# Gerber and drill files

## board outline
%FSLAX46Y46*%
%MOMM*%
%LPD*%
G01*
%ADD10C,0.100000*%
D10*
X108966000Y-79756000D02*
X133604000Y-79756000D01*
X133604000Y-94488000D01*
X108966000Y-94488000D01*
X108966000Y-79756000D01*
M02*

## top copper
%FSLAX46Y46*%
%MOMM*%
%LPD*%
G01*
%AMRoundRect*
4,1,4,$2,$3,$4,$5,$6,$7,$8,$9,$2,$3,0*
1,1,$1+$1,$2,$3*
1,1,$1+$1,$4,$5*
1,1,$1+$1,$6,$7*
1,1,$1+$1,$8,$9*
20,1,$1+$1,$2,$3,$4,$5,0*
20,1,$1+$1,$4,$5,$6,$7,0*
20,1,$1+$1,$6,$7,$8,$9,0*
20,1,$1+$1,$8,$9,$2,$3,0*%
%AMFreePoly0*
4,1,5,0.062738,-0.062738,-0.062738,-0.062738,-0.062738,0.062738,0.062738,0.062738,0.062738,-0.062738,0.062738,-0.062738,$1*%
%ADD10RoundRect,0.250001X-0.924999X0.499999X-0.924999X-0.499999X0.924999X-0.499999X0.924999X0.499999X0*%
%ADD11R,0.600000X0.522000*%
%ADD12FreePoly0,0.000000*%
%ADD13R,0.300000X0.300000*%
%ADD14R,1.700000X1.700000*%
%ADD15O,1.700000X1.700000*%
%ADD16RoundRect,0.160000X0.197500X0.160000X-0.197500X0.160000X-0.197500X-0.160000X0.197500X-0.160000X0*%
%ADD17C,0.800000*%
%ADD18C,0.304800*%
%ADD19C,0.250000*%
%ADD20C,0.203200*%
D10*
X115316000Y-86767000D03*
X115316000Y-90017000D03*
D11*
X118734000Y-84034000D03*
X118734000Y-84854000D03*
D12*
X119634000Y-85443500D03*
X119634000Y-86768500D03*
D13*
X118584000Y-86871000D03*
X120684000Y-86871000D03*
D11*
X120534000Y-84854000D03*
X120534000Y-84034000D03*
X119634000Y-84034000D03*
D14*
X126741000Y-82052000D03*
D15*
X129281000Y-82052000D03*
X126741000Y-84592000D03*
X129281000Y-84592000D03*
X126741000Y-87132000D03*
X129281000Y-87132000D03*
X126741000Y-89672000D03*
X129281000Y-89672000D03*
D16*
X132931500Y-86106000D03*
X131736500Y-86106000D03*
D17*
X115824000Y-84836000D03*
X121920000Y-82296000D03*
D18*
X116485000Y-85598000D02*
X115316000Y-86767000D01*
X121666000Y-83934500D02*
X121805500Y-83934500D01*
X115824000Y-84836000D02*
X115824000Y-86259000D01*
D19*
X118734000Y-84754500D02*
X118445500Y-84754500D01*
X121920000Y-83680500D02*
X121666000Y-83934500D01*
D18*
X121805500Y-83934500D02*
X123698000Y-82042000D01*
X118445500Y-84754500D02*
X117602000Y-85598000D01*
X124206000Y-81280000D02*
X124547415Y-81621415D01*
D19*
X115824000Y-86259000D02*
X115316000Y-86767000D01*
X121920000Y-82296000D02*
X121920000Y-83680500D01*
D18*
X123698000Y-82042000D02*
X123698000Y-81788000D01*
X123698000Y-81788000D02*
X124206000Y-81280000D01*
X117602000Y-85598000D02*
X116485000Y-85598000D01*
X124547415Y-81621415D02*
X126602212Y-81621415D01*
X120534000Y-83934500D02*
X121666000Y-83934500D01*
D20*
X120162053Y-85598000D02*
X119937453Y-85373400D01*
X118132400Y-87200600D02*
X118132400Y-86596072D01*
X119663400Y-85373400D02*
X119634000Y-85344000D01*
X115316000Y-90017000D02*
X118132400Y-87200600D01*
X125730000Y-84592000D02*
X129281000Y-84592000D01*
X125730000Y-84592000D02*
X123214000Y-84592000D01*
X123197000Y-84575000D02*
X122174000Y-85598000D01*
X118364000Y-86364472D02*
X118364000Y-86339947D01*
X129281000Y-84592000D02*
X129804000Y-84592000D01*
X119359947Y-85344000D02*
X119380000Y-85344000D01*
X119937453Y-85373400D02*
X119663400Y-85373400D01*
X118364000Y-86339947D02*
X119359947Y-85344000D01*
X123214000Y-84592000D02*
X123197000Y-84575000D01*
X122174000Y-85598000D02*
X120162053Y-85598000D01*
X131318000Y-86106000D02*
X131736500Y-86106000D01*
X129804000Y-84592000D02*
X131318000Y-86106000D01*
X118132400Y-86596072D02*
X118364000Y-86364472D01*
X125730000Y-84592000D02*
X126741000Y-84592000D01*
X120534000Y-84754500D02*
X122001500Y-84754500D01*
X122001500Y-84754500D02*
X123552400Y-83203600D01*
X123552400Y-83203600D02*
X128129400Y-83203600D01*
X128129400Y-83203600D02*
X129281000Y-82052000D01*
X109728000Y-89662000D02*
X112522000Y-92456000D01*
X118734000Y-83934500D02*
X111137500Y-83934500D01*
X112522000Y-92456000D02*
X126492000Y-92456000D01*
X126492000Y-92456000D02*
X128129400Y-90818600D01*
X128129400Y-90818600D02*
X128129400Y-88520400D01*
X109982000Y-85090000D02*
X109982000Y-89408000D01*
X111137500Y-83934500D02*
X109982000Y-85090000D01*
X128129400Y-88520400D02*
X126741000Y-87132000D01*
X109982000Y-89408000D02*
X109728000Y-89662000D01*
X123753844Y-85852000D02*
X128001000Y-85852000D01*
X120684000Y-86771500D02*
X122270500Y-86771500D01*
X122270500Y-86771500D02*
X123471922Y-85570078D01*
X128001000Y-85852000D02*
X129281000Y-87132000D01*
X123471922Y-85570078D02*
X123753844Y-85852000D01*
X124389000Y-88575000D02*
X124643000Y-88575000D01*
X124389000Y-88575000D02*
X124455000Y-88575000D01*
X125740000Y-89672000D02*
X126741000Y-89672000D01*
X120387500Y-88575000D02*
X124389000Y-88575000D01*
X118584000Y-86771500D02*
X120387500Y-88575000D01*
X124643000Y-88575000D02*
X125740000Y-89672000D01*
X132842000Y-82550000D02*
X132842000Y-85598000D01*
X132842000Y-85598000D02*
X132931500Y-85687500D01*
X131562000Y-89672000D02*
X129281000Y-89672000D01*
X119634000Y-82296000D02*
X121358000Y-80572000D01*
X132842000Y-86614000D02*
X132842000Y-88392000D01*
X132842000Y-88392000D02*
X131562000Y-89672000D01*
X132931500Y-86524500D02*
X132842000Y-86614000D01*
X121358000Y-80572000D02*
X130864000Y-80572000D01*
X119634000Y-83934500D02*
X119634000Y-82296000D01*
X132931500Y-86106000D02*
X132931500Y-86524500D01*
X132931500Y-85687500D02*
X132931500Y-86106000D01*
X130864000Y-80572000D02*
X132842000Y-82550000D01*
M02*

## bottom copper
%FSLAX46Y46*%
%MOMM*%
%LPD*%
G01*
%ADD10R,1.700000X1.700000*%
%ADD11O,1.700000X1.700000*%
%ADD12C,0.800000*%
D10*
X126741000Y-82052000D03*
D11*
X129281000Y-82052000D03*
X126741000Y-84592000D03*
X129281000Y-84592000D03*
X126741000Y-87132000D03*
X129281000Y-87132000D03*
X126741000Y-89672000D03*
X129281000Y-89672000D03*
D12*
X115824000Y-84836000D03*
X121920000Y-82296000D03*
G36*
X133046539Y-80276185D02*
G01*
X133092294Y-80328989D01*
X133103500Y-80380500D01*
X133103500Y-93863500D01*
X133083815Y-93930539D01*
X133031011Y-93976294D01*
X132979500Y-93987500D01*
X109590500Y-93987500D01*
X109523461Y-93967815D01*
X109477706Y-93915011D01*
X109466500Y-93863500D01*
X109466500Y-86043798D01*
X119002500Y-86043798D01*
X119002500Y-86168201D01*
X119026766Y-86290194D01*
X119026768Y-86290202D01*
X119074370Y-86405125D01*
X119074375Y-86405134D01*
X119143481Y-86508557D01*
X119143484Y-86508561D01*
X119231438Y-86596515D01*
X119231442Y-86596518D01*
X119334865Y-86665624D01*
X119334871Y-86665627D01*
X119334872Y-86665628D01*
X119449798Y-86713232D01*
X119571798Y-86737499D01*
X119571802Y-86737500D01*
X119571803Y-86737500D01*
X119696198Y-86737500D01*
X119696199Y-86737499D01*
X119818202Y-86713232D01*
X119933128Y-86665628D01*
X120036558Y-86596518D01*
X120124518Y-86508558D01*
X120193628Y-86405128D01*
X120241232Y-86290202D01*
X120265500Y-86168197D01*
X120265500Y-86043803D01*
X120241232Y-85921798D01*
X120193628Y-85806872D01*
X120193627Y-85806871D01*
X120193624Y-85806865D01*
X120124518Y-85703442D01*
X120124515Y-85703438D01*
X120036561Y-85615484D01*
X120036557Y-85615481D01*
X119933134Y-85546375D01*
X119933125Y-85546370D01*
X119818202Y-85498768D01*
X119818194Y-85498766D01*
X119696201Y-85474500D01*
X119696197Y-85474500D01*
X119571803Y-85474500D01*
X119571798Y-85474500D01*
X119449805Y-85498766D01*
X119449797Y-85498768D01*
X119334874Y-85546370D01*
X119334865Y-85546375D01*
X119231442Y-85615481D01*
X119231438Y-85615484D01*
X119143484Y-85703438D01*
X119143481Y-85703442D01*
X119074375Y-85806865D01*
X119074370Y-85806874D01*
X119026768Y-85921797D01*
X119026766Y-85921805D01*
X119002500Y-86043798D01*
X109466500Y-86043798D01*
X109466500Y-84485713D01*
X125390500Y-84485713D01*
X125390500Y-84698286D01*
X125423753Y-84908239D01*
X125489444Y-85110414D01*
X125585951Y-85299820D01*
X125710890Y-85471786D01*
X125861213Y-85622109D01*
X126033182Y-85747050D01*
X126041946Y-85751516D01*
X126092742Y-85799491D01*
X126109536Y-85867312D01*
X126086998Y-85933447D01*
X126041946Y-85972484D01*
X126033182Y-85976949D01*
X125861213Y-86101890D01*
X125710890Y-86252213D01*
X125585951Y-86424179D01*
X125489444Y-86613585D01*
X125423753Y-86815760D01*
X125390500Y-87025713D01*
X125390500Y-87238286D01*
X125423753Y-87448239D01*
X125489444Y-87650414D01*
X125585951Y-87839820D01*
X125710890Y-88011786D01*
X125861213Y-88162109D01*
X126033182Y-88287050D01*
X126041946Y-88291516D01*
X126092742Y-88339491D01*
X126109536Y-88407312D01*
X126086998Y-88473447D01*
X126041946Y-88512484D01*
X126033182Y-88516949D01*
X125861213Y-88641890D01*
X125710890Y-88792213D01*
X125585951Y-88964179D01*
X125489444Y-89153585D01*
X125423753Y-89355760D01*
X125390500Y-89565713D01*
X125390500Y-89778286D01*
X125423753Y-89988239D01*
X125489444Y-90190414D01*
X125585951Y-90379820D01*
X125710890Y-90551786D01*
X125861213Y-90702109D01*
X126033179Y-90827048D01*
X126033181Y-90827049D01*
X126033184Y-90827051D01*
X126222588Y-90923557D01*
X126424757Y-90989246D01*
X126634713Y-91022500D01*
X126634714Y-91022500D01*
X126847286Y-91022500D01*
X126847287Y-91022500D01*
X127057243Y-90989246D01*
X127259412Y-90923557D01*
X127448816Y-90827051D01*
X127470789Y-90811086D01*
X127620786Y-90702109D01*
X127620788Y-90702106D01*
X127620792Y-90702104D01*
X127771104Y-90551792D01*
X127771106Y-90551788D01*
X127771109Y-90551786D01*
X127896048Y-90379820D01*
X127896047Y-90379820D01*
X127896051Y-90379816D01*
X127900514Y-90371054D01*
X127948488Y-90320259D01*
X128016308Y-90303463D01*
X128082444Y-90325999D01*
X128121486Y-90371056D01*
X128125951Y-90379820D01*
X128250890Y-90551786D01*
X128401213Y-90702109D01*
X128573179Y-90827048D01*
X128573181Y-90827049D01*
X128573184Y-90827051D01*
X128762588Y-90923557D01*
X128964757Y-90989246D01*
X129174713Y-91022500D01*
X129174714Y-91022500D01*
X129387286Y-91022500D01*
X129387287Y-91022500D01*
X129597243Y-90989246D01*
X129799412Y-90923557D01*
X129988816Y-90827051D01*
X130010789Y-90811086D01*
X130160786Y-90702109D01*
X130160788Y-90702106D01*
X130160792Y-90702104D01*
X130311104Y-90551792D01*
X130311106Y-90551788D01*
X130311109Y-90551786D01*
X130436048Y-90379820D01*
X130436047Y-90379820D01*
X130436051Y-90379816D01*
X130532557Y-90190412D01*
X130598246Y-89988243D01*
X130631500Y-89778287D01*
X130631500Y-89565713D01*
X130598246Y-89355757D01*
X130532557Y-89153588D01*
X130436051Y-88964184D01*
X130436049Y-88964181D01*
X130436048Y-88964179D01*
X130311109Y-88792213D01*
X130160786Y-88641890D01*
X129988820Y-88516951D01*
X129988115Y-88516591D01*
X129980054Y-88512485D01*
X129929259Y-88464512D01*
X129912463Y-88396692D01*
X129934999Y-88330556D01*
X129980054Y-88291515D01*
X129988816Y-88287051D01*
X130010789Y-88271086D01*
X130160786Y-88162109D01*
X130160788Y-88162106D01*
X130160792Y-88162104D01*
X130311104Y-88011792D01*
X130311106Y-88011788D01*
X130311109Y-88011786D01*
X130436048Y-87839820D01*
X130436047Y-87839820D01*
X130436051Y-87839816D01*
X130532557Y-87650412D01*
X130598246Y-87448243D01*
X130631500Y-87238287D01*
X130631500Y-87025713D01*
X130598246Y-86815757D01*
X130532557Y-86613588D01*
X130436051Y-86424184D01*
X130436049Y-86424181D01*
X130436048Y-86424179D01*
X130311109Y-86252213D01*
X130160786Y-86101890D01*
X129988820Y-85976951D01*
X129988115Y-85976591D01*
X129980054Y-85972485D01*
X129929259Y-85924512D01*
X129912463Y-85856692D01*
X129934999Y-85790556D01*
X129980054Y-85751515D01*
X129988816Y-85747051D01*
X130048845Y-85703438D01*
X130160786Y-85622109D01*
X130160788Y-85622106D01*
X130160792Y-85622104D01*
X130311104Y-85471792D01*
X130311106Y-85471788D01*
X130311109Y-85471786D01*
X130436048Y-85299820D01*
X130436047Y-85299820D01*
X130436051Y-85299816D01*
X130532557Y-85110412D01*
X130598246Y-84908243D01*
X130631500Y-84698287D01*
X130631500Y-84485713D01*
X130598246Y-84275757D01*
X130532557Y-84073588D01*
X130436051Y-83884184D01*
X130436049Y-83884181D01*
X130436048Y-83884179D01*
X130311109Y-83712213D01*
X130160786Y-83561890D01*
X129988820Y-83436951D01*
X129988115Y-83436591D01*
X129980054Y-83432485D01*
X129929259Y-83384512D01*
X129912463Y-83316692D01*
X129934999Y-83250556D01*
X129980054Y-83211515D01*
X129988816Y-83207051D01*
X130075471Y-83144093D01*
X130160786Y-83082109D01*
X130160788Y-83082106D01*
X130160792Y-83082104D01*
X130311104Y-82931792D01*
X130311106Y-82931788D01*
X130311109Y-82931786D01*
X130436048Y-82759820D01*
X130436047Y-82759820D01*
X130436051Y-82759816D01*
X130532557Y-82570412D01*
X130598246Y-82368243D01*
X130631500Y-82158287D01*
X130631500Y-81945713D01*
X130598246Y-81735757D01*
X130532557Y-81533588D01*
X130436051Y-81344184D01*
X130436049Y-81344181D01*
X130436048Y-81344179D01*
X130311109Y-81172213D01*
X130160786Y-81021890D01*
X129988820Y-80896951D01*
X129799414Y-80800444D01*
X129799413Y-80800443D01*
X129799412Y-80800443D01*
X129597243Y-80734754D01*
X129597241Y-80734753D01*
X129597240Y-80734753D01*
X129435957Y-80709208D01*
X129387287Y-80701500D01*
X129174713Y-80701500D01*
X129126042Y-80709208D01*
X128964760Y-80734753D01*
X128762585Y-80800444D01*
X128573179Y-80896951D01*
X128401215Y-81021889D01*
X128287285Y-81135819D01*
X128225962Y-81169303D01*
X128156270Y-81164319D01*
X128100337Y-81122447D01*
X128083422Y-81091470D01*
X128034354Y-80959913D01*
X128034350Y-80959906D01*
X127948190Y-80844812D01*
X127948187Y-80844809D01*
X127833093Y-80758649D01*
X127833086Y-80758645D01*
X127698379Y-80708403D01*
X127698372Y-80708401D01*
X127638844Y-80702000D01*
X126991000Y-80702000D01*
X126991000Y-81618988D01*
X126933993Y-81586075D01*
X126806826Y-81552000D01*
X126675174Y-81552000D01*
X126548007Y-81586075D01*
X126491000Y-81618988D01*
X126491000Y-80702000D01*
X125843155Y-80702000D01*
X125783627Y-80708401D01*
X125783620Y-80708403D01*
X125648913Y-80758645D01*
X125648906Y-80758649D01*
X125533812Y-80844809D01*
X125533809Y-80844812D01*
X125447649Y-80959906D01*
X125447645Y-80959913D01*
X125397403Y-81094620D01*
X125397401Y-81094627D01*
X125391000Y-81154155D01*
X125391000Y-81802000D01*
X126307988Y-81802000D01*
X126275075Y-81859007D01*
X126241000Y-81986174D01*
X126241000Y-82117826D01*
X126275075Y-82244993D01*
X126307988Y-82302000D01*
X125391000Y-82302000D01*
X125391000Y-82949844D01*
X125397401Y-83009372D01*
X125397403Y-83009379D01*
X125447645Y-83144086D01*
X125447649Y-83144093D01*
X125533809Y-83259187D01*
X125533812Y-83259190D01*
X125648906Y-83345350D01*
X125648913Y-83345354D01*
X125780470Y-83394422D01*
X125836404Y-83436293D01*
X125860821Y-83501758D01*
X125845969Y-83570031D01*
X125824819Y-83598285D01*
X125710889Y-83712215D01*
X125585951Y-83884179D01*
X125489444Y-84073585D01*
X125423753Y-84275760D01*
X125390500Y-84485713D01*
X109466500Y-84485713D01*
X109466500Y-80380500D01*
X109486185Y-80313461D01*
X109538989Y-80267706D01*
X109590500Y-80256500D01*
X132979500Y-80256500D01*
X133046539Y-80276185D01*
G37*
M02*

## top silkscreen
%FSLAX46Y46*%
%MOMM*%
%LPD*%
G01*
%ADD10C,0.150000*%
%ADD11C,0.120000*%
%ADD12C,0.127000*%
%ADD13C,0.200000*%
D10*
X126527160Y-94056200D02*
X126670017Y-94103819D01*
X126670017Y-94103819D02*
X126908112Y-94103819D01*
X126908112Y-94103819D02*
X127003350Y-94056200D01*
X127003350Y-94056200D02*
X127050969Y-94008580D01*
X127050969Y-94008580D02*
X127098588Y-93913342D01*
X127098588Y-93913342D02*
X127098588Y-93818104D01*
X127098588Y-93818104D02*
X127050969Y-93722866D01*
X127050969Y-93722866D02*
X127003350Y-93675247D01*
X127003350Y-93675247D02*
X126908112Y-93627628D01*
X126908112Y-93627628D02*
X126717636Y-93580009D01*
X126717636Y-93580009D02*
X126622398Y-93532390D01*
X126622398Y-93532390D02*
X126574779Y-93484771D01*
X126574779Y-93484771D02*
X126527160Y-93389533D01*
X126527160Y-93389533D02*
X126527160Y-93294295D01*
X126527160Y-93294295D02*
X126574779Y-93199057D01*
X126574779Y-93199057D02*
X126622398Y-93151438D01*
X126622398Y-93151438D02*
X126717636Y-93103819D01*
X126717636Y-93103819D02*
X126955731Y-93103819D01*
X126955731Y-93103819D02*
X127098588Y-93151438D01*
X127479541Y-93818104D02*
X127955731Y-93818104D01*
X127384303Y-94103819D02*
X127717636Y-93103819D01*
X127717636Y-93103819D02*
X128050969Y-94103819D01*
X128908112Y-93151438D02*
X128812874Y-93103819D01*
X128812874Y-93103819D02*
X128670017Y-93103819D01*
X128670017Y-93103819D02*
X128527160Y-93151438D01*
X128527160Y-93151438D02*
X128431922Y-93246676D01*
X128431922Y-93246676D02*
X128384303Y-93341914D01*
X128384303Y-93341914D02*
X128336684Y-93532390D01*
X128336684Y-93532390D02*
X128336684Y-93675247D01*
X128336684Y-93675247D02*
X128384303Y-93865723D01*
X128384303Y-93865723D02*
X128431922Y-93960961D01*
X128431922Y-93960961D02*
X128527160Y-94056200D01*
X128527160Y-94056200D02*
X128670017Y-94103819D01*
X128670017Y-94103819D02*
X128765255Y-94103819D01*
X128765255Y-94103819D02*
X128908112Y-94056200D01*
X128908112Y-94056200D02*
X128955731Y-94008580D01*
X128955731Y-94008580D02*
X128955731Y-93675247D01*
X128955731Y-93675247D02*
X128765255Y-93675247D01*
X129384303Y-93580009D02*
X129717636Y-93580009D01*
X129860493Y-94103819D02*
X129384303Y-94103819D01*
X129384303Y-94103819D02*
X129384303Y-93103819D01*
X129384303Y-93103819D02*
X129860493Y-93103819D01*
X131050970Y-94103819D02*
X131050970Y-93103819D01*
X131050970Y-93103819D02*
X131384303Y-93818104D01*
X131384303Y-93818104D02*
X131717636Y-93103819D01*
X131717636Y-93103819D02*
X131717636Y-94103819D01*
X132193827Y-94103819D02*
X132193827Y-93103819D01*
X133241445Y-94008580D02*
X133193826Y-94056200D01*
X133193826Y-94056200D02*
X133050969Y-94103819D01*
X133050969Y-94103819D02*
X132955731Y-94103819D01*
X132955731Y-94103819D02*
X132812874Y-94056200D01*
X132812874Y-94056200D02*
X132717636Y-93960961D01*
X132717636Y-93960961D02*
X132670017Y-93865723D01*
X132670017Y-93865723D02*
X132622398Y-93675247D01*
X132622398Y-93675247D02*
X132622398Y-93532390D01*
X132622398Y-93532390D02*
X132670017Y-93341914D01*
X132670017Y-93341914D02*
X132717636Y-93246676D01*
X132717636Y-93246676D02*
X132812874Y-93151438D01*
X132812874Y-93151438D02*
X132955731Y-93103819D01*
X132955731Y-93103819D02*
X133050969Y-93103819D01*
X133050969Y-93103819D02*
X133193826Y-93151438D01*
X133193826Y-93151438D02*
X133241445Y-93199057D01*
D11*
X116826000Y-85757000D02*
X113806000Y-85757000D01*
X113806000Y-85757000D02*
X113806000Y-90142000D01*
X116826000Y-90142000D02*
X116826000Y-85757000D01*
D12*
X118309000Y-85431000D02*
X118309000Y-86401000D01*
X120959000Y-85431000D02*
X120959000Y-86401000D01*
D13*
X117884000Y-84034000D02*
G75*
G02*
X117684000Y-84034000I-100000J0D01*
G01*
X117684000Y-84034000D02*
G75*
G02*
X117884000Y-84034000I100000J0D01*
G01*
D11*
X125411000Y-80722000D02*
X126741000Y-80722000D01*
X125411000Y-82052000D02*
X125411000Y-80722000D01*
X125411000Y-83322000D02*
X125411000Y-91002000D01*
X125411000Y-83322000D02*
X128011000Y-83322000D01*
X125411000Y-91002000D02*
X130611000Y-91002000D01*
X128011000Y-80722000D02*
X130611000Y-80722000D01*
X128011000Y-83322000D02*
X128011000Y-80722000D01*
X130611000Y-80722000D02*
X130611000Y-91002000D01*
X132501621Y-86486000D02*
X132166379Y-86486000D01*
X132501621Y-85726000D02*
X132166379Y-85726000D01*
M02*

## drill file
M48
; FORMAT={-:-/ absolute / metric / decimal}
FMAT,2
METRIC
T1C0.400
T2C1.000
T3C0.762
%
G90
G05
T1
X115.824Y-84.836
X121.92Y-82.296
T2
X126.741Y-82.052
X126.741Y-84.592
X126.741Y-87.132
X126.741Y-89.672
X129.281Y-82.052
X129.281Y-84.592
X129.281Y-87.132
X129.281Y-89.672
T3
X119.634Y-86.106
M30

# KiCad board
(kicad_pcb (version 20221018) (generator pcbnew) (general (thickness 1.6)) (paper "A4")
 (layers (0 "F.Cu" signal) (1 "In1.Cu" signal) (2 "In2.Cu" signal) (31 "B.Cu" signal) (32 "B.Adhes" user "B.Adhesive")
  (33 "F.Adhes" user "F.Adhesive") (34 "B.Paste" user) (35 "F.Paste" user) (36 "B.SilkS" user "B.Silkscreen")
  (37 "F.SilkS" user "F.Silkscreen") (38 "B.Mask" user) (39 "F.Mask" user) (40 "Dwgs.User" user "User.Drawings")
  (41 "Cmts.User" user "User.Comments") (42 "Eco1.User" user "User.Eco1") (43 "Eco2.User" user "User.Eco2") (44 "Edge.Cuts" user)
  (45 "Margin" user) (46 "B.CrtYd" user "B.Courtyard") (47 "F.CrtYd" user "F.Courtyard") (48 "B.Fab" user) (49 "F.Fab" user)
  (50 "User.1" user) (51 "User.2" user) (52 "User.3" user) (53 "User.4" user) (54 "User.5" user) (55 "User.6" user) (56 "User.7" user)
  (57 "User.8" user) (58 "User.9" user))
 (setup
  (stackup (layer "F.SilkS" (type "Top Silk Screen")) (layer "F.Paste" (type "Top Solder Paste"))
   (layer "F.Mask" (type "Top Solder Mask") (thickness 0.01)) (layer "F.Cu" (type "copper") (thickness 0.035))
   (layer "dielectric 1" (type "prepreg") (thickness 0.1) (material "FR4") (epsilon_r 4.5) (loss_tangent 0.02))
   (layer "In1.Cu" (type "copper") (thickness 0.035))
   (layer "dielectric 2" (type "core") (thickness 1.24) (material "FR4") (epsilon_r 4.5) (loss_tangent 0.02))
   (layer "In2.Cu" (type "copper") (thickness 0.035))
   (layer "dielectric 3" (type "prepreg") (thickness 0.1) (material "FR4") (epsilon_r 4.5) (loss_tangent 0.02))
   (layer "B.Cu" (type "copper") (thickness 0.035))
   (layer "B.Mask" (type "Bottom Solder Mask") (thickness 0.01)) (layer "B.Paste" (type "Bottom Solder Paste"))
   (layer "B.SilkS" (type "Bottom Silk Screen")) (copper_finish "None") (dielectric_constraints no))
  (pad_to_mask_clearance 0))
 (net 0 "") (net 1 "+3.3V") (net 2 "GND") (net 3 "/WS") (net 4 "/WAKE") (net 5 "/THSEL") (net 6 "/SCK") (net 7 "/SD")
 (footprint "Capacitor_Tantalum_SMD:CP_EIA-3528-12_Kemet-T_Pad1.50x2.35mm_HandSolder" (layer "F.Cu") (at 115.316 88.392 -90)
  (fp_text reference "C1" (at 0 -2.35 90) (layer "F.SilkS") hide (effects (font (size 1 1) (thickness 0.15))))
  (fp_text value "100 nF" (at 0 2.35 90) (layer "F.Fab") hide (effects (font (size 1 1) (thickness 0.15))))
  (fp_line (start -2.635 -1.51) (end -2.635 1.51) (stroke (width 0.12) (type solid)) (layer "F.SilkS"))
  (fp_line (start -2.635 1.51) (end 1.75 1.51) (stroke (width 0.12) (type solid)) (layer "F.SilkS"))
  (fp_line (start 1.75 -1.51) (end -2.635 -1.51) (stroke (width 0.12) (type solid)) (layer "F.SilkS"))
  (pad "1" smd roundrect (at -1.625 0 270) (size 1.5 2.35) (layers "F.Cu" "F.Paste" "F.Mask") (roundrect_rratio 0.166667) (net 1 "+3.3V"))
  (pad "2" smd roundrect (at 1.625 0 270) (size 1.5 2.35) (layers "F.Cu" "F.Paste" "F.Mask") (roundrect_rratio 0.166667) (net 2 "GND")))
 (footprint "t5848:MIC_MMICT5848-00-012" (layer "F.Cu") (at 119.634 85.396)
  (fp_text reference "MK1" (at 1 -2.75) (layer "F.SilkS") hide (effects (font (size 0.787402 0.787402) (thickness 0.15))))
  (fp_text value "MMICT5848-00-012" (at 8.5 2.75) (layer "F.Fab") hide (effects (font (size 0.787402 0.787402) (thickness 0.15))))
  (fp_line (start -1.325 0.035) (end -1.325 1.005) (stroke (width 0.127) (type solid)) (layer "F.SilkS"))
  (fp_line (start 1.325 0.035) (end 1.325 1.005) (stroke (width 0.127) (type solid)) (layer "F.SilkS"))
  (fp_circle (center -1.85 -1.362) (end -1.75 -1.362) (stroke (width 0.2) (type solid)) (fill none) (layer "F.SilkS"))
  (pad "" np_thru_hole circle (at 0 0.71) (size 0.001 0.001) (drill 0.762) (layers "F&B.Cu" "*.Mask"))
  (pad "1" smd rect (at -0.9 -1.362) (size 0.6 0.522) (layers "F.Cu") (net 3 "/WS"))
  (pad "2" smd rect (at -0.9 -0.542) (size 0.6 0.522) (layers "F.Cu") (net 1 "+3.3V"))
  (pad "3_1" smd custom (at 0 0.0475) (size 0.125476 0.125476) (layers "F.Cu") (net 2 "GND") (options (clearance outline) (anchor rect))
   (primitives))
  (pad "3_2" smd custom (at 0 1.3725) (size 0.125476 0.125476) (layers "F.Cu") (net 2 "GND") (options (clearance outline) (anchor rect))
   (primitives))
  (pad "4" smd rect (at -1.05 1.475) (size 0.3 0.3) (layers "F.Cu") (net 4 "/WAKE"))
  (pad "5" smd rect (at 1.05 1.475) (size 0.3 0.3) (layers "F.Cu") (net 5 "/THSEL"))
  (pad "6" smd rect (at 0.9 -0.542) (size 0.6 0.522) (layers "F.Cu") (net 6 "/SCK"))
  (pad "7" smd rect (at 0.9 -1.362) (size 0.6 0.522) (layers "F.Cu") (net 1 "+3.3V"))
  (pad "8" smd rect (at 0 -1.362) (size 0.6 0.522) (layers "F.Cu") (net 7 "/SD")))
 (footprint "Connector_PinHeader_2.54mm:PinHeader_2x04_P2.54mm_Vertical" (layer "F.Cu") (at 126.741 82.052)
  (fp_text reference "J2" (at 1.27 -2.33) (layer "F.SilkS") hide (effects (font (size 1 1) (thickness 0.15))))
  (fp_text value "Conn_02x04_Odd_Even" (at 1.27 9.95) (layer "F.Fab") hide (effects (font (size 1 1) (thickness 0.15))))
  (fp_line (start -1.33 -1.33) (end 0 -1.33) (stroke (width 0.12) (type solid)) (layer "F.SilkS"))
  (fp_line (start -1.33 0) (end -1.33 -1.33) (stroke (width 0.12) (type solid)) (layer "F.SilkS"))
  (fp_line (start -1.33 1.27) (end -1.33 8.95) (stroke (width 0.12) (type solid)) (layer "F.SilkS"))
  (fp_line (start -1.33 1.27) (end 1.27 1.27) (stroke (width 0.12) (type solid)) (layer "F.SilkS"))
  (fp_line (start -1.33 8.95) (end 3.87 8.95) (stroke (width 0.12) (type solid)) (layer "F.SilkS"))
  (fp_line (start 1.27 -1.33) (end 3.87 -1.33) (stroke (width 0.12) (type solid)) (layer "F.SilkS"))
  (fp_line (start 1.27 1.27) (end 1.27 -1.33) (stroke (width 0.12) (type solid)) (layer "F.SilkS"))
  (fp_line (start 3.87 -1.33) (end 3.87 8.95) (stroke (width 0.12) (type solid)) (layer "F.SilkS"))
  (pad "1" thru_hole rect (at 0 0) (size 1.7 1.7) (drill 1) (layers "*.Cu" "*.Mask") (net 1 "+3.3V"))
  (pad "2" thru_hole oval (at 2.54 0) (size 1.7 1.7) (drill 1) (layers "*.Cu" "*.Mask") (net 6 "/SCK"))
  (pad "3" thru_hole oval (at 0 2.54) (size 1.7 1.7) (drill 1) (layers "*.Cu" "*.Mask") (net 2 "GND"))
  (pad "4" thru_hole oval (at 2.54 2.54) (size 1.7 1.7) (drill 1) (layers "*.Cu" "*.Mask") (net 2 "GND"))
  (pad "5" thru_hole oval (at 0 5.08) (size 1.7 1.7) (drill 1) (layers "*.Cu" "*.Mask") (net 3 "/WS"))
  (pad "6" thru_hole oval (at 2.54 5.08) (size 1.7 1.7) (drill 1) (layers "*.Cu" "*.Mask") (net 5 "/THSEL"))
  (pad "7" thru_hole oval (at 0 7.62) (size 1.7 1.7) (drill 1) (layers "*.Cu" "*.Mask") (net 4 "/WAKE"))
  (pad "8" thru_hole oval (at 2.54 7.62) (size 1.7 1.7) (drill 1) (layers "*.Cu" "*.Mask") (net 7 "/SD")))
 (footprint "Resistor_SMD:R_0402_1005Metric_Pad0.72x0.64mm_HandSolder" (layer "F.Cu") (at 132.334 86.106 180)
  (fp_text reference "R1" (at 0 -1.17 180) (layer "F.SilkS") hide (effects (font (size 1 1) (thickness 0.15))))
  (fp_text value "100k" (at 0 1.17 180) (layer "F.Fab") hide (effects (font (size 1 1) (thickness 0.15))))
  (fp_line (start -0.167621 -0.38) (end 0.167621 -0.38) (stroke (width 0.12) (type solid)) (layer "F.SilkS"))
  (fp_line (start -0.167621 0.38) (end 0.167621 0.38) (stroke (width 0.12) (type solid)) (layer "F.SilkS"))
  (pad "1" smd roundrect (at -0.5975 0 180) (size 0.715 0.64) (layers "F.Cu" "F.Paste" "F.Mask") (roundrect_rratio 0.25) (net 7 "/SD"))
  (pad "2" smd roundrect (at 0.5975 0 180) (size 0.715 0.64) (layers "F.Cu" "F.Paste" "F.Mask") (roundrect_rratio 0.25) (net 2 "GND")))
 (gr_rect (start 108.966 79.756) (end 133.604 94.488) (stroke (width 0.1) (type default)) (fill none) (layer "Edge.Cuts"))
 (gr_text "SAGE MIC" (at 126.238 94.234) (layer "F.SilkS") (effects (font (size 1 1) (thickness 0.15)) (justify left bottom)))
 (segment (start 116.485 85.598) (end 115.316 86.767) (width 0.3048) (layer "F.Cu") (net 1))
 (segment (start 121.666 83.9345) (end 121.8055 83.9345) (width 0.3048) (layer "F.Cu") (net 1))
 (segment (start 115.824 84.836) (end 115.824 86.259) (width 0.3048) (layer "F.Cu") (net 1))
 (segment (start 118.734 84.7545) (end 118.4455 84.7545) (width 0.25) (layer "F.Cu") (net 1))
 (segment (start 121.92 83.6805) (end 121.666 83.9345) (width 0.25) (layer "F.Cu") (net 1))
 (segment (start 121.8055 83.9345) (end 123.698 82.042) (width 0.3048) (layer "F.Cu") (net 1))
 (segment (start 118.4455 84.7545) (end 117.602 85.598) (width 0.3048) (layer "F.Cu") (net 1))
 (segment (start 124.206 81.28) (end 124.547415 81.621415) (width 0.3048) (layer "F.Cu") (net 1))
 (segment (start 115.824 86.259) (end 115.316 86.767) (width 0.25) (layer "F.Cu") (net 1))
 (segment (start 121.92 82.296) (end 121.92 83.6805) (width 0.25) (layer "F.Cu") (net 1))
 (segment (start 123.698 82.042) (end 123.698 81.788) (width 0.3048) (layer "F.Cu") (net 1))
 (segment (start 123.698 81.788) (end 124.206 81.28) (width 0.3048) (layer "F.Cu") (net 1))
 (segment (start 117.602 85.598) (end 116.485 85.598) (width 0.3048) (layer "F.Cu") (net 1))
 (segment (start 124.547415 81.621415) (end 126.602212 81.621415) (width 0.3048) (layer "F.Cu") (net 1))
 (segment (start 120.534 83.9345) (end 121.666 83.9345) (width 0.3048) (layer "F.Cu") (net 1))
 (via (at 115.824 84.836) (size 0.8) (drill 0.4) (layers "F.Cu" "B.Cu") (free) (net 1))
 (via (at 121.92 82.296) (size 0.8) (drill 0.4) (layers "F.Cu" "B.Cu") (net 1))
 (segment (start 120.162053 85.598) (end 119.937453 85.3734) (width 0.2032) (layer "F.Cu") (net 2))
 (segment (start 118.1324 87.2006) (end 118.1324 86.596072) (width 0.2032) (layer "F.Cu") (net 2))
 (segment (start 119.6634 85.3734) (end 119.634 85.344) (width 0.2032) (layer "F.Cu") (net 2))
 (segment (start 115.316 90.017) (end 118.1324 87.2006) (width 0.2032) (layer "F.Cu") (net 2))
 (segment (start 125.73 84.592) (end 129.281 84.592) (width 0.2032) (layer "F.Cu") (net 2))
 (segment (start 125.73 84.592) (end 123.214 84.592) (width 0.2032) (layer "F.Cu") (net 2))
 (segment (start 123.197 84.575) (end 122.174 85.598) (width 0.2032) (layer "F.Cu") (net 2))
 (segment (start 118.364 86.364472) (end 118.364 86.339947) (width 0.2032) (layer "F.Cu") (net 2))
 (segment (start 129.281 84.592) (end 129.804 84.592) (width 0.2032) (layer "F.Cu") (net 2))
 (segment (start 119.359947 85.344) (end 119.38 85.344) (width 0.2032) (layer "F.Cu") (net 2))
 (segment (start 119.937453 85.3734) (end 119.6634 85.3734) (width 0.2032) (layer "F.Cu") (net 2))
 (segment (start 118.364 86.339947) (end 119.359947 85.344) (width 0.2032) (layer "F.Cu") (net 2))
 (segment (start 123.214 84.592) (end 123.197 84.575) (width 0.2032) (layer "F.Cu") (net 2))
 (segment (start 122.174 85.598) (end 120.162053 85.598) (width 0.2032) (layer "F.Cu") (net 2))
 (segment (start 131.318 86.106) (end 131.7365 86.106) (width 0.2032) (layer "F.Cu") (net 2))
 (segment (start 129.804 84.592) (end 131.318 86.106) (width 0.2032) (layer "F.Cu") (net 2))
 (segment (start 118.1324 86.596072) (end 118.364 86.364472) (width 0.2032) (layer "F.Cu") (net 2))
 (segment (start 125.73 84.592) (end 126.741 84.592) (width 0.2032) (layer "F.Cu") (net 2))
 (segment (start 120.534 84.7545) (end 122.0015 84.7545) (width 0.2032) (layer "F.Cu") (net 6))
 (segment (start 122.0015 84.7545) (end 123.5524 83.2036) (width 0.2032) (layer "F.Cu") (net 6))
 (segment (start 123.5524 83.2036) (end 128.1294 83.2036) (width 0.2032) (layer "F.Cu") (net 6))
 (segment (start 128.1294 83.2036) (end 129.281 82.052) (width 0.2032) (layer "F.Cu") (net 6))
 (segment (start 109.728 89.662) (end 112.522 92.456) (width 0.2032) (layer "F.Cu") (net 3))
 (segment (start 118.734 83.9345) (end 111.1375 83.9345) (width 0.2032) (layer "F.Cu") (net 3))
 (segment (start 112.522 92.456) (end 126.492 92.456) (width 0.2032) (layer "F.Cu") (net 3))
 (segment (start 126.492 92.456) (end 128.1294 90.8186) (width 0.2032) (layer "F.Cu") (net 3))
 (segment (start 128.1294 90.8186) (end 128.1294 88.5204) (width 0.2032) (layer "F.Cu") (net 3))
 (segment (start 109.982 85.09) (end 109.982 89.408) (width 0.2032) (layer "F.Cu") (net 3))
 (segment (start 111.1375 83.9345) (end 109.982 85.09) (width 0.2032) (layer "F.Cu") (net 3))
 (segment (start 128.1294 88.5204) (end 126.741 87.132) (width 0.2032) (layer "F.Cu") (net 3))
 (segment (start 109.982 89.408) (end 109.728 89.662) (width 0.2032) (layer "F.Cu") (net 3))
 (segment (start 123.753844 85.852) (end 128.001 85.852) (width 0.2032) (layer "F.Cu") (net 5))
 (segment (start 120.684 86.7715) (end 122.2705 86.7715) (width 0.2032) (layer "F.Cu") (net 5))
 (segment (start 122.2705 86.7715) (end 123.471922 85.570078) (width 0.2032) (layer "F.Cu") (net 5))
 (segment (start 128.001 85.852) (end 129.281 87.132) (width 0.2032) (layer "F.Cu") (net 5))
 (segment (start 123.471922 85.570078) (end 123.753844 85.852) (width 0.2032) (layer "F.Cu") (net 5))
 (segment (start 124.389 88.575) (end 124.643 88.575) (width 0.2032) (layer "F.Cu") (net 4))
 (segment (start 124.389 88.575) (end 124.455 88.575) (width 0.2032) (layer "F.Cu") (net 4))
 (segment (start 125.74 89.672) (end 126.741 89.672) (width 0.2032) (layer "F.Cu") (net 4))
 (segment (start 120.3875 88.575) (end 124.389 88.575) (width 0.2032) (layer "F.Cu") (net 4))
 (segment (start 118.584 86.7715) (end 120.3875 88.575) (width 0.2032) (layer "F.Cu") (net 4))
 (segment (start 124.643 88.575) (end 125.74 89.672) (width 0.2032) (layer "F.Cu") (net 4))
 (segment (start 132.842 82.55) (end 132.842 85.598) (width 0.2032) (layer "F.Cu") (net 7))
 (segment (start 132.842 85.598) (end 132.9315 85.6875) (width 0.2032) (layer "F.Cu") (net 7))
 (segment (start 131.562 89.672) (end 129.281 89.672) (width 0.2032) (layer "F.Cu") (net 7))
 (segment (start 119.634 82.296) (end 121.358 80.572) (width 0.2032) (layer "F.Cu") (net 7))
 (segment (start 132.842 86.614) (end 132.842 88.392) (width 0.2032) (layer "F.Cu") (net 7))
 (segment (start 132.842 88.392) (end 131.562 89.672) (width 0.2032) (layer "F.Cu") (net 7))
 (segment (start 132.9315 86.5245) (end 132.842 86.614) (width 0.2032) (layer "F.Cu") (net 7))
 (segment (start 121.358 80.572) (end 130.864 80.572) (width 0.2032) (layer "F.Cu") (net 7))
 (segment (start 119.634 83.9345) (end 119.634 82.296) (width 0.2032) (layer "F.Cu") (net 7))
 (segment (start 132.9315 86.106) (end 132.9315 86.5245) (width 0.2032) (layer "F.Cu") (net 7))
 (segment (start 132.9315 85.6875) (end 132.9315 86.106) (width 0.2032) (layer "F.Cu") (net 7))
 (segment (start 130.864 80.572) (end 132.842 82.55) (width 0.2032) (layer "F.Cu") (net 7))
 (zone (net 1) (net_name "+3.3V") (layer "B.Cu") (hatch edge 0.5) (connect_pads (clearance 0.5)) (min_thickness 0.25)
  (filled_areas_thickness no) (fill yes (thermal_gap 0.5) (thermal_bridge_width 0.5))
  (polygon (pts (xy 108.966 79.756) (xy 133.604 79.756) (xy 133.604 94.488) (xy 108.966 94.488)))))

